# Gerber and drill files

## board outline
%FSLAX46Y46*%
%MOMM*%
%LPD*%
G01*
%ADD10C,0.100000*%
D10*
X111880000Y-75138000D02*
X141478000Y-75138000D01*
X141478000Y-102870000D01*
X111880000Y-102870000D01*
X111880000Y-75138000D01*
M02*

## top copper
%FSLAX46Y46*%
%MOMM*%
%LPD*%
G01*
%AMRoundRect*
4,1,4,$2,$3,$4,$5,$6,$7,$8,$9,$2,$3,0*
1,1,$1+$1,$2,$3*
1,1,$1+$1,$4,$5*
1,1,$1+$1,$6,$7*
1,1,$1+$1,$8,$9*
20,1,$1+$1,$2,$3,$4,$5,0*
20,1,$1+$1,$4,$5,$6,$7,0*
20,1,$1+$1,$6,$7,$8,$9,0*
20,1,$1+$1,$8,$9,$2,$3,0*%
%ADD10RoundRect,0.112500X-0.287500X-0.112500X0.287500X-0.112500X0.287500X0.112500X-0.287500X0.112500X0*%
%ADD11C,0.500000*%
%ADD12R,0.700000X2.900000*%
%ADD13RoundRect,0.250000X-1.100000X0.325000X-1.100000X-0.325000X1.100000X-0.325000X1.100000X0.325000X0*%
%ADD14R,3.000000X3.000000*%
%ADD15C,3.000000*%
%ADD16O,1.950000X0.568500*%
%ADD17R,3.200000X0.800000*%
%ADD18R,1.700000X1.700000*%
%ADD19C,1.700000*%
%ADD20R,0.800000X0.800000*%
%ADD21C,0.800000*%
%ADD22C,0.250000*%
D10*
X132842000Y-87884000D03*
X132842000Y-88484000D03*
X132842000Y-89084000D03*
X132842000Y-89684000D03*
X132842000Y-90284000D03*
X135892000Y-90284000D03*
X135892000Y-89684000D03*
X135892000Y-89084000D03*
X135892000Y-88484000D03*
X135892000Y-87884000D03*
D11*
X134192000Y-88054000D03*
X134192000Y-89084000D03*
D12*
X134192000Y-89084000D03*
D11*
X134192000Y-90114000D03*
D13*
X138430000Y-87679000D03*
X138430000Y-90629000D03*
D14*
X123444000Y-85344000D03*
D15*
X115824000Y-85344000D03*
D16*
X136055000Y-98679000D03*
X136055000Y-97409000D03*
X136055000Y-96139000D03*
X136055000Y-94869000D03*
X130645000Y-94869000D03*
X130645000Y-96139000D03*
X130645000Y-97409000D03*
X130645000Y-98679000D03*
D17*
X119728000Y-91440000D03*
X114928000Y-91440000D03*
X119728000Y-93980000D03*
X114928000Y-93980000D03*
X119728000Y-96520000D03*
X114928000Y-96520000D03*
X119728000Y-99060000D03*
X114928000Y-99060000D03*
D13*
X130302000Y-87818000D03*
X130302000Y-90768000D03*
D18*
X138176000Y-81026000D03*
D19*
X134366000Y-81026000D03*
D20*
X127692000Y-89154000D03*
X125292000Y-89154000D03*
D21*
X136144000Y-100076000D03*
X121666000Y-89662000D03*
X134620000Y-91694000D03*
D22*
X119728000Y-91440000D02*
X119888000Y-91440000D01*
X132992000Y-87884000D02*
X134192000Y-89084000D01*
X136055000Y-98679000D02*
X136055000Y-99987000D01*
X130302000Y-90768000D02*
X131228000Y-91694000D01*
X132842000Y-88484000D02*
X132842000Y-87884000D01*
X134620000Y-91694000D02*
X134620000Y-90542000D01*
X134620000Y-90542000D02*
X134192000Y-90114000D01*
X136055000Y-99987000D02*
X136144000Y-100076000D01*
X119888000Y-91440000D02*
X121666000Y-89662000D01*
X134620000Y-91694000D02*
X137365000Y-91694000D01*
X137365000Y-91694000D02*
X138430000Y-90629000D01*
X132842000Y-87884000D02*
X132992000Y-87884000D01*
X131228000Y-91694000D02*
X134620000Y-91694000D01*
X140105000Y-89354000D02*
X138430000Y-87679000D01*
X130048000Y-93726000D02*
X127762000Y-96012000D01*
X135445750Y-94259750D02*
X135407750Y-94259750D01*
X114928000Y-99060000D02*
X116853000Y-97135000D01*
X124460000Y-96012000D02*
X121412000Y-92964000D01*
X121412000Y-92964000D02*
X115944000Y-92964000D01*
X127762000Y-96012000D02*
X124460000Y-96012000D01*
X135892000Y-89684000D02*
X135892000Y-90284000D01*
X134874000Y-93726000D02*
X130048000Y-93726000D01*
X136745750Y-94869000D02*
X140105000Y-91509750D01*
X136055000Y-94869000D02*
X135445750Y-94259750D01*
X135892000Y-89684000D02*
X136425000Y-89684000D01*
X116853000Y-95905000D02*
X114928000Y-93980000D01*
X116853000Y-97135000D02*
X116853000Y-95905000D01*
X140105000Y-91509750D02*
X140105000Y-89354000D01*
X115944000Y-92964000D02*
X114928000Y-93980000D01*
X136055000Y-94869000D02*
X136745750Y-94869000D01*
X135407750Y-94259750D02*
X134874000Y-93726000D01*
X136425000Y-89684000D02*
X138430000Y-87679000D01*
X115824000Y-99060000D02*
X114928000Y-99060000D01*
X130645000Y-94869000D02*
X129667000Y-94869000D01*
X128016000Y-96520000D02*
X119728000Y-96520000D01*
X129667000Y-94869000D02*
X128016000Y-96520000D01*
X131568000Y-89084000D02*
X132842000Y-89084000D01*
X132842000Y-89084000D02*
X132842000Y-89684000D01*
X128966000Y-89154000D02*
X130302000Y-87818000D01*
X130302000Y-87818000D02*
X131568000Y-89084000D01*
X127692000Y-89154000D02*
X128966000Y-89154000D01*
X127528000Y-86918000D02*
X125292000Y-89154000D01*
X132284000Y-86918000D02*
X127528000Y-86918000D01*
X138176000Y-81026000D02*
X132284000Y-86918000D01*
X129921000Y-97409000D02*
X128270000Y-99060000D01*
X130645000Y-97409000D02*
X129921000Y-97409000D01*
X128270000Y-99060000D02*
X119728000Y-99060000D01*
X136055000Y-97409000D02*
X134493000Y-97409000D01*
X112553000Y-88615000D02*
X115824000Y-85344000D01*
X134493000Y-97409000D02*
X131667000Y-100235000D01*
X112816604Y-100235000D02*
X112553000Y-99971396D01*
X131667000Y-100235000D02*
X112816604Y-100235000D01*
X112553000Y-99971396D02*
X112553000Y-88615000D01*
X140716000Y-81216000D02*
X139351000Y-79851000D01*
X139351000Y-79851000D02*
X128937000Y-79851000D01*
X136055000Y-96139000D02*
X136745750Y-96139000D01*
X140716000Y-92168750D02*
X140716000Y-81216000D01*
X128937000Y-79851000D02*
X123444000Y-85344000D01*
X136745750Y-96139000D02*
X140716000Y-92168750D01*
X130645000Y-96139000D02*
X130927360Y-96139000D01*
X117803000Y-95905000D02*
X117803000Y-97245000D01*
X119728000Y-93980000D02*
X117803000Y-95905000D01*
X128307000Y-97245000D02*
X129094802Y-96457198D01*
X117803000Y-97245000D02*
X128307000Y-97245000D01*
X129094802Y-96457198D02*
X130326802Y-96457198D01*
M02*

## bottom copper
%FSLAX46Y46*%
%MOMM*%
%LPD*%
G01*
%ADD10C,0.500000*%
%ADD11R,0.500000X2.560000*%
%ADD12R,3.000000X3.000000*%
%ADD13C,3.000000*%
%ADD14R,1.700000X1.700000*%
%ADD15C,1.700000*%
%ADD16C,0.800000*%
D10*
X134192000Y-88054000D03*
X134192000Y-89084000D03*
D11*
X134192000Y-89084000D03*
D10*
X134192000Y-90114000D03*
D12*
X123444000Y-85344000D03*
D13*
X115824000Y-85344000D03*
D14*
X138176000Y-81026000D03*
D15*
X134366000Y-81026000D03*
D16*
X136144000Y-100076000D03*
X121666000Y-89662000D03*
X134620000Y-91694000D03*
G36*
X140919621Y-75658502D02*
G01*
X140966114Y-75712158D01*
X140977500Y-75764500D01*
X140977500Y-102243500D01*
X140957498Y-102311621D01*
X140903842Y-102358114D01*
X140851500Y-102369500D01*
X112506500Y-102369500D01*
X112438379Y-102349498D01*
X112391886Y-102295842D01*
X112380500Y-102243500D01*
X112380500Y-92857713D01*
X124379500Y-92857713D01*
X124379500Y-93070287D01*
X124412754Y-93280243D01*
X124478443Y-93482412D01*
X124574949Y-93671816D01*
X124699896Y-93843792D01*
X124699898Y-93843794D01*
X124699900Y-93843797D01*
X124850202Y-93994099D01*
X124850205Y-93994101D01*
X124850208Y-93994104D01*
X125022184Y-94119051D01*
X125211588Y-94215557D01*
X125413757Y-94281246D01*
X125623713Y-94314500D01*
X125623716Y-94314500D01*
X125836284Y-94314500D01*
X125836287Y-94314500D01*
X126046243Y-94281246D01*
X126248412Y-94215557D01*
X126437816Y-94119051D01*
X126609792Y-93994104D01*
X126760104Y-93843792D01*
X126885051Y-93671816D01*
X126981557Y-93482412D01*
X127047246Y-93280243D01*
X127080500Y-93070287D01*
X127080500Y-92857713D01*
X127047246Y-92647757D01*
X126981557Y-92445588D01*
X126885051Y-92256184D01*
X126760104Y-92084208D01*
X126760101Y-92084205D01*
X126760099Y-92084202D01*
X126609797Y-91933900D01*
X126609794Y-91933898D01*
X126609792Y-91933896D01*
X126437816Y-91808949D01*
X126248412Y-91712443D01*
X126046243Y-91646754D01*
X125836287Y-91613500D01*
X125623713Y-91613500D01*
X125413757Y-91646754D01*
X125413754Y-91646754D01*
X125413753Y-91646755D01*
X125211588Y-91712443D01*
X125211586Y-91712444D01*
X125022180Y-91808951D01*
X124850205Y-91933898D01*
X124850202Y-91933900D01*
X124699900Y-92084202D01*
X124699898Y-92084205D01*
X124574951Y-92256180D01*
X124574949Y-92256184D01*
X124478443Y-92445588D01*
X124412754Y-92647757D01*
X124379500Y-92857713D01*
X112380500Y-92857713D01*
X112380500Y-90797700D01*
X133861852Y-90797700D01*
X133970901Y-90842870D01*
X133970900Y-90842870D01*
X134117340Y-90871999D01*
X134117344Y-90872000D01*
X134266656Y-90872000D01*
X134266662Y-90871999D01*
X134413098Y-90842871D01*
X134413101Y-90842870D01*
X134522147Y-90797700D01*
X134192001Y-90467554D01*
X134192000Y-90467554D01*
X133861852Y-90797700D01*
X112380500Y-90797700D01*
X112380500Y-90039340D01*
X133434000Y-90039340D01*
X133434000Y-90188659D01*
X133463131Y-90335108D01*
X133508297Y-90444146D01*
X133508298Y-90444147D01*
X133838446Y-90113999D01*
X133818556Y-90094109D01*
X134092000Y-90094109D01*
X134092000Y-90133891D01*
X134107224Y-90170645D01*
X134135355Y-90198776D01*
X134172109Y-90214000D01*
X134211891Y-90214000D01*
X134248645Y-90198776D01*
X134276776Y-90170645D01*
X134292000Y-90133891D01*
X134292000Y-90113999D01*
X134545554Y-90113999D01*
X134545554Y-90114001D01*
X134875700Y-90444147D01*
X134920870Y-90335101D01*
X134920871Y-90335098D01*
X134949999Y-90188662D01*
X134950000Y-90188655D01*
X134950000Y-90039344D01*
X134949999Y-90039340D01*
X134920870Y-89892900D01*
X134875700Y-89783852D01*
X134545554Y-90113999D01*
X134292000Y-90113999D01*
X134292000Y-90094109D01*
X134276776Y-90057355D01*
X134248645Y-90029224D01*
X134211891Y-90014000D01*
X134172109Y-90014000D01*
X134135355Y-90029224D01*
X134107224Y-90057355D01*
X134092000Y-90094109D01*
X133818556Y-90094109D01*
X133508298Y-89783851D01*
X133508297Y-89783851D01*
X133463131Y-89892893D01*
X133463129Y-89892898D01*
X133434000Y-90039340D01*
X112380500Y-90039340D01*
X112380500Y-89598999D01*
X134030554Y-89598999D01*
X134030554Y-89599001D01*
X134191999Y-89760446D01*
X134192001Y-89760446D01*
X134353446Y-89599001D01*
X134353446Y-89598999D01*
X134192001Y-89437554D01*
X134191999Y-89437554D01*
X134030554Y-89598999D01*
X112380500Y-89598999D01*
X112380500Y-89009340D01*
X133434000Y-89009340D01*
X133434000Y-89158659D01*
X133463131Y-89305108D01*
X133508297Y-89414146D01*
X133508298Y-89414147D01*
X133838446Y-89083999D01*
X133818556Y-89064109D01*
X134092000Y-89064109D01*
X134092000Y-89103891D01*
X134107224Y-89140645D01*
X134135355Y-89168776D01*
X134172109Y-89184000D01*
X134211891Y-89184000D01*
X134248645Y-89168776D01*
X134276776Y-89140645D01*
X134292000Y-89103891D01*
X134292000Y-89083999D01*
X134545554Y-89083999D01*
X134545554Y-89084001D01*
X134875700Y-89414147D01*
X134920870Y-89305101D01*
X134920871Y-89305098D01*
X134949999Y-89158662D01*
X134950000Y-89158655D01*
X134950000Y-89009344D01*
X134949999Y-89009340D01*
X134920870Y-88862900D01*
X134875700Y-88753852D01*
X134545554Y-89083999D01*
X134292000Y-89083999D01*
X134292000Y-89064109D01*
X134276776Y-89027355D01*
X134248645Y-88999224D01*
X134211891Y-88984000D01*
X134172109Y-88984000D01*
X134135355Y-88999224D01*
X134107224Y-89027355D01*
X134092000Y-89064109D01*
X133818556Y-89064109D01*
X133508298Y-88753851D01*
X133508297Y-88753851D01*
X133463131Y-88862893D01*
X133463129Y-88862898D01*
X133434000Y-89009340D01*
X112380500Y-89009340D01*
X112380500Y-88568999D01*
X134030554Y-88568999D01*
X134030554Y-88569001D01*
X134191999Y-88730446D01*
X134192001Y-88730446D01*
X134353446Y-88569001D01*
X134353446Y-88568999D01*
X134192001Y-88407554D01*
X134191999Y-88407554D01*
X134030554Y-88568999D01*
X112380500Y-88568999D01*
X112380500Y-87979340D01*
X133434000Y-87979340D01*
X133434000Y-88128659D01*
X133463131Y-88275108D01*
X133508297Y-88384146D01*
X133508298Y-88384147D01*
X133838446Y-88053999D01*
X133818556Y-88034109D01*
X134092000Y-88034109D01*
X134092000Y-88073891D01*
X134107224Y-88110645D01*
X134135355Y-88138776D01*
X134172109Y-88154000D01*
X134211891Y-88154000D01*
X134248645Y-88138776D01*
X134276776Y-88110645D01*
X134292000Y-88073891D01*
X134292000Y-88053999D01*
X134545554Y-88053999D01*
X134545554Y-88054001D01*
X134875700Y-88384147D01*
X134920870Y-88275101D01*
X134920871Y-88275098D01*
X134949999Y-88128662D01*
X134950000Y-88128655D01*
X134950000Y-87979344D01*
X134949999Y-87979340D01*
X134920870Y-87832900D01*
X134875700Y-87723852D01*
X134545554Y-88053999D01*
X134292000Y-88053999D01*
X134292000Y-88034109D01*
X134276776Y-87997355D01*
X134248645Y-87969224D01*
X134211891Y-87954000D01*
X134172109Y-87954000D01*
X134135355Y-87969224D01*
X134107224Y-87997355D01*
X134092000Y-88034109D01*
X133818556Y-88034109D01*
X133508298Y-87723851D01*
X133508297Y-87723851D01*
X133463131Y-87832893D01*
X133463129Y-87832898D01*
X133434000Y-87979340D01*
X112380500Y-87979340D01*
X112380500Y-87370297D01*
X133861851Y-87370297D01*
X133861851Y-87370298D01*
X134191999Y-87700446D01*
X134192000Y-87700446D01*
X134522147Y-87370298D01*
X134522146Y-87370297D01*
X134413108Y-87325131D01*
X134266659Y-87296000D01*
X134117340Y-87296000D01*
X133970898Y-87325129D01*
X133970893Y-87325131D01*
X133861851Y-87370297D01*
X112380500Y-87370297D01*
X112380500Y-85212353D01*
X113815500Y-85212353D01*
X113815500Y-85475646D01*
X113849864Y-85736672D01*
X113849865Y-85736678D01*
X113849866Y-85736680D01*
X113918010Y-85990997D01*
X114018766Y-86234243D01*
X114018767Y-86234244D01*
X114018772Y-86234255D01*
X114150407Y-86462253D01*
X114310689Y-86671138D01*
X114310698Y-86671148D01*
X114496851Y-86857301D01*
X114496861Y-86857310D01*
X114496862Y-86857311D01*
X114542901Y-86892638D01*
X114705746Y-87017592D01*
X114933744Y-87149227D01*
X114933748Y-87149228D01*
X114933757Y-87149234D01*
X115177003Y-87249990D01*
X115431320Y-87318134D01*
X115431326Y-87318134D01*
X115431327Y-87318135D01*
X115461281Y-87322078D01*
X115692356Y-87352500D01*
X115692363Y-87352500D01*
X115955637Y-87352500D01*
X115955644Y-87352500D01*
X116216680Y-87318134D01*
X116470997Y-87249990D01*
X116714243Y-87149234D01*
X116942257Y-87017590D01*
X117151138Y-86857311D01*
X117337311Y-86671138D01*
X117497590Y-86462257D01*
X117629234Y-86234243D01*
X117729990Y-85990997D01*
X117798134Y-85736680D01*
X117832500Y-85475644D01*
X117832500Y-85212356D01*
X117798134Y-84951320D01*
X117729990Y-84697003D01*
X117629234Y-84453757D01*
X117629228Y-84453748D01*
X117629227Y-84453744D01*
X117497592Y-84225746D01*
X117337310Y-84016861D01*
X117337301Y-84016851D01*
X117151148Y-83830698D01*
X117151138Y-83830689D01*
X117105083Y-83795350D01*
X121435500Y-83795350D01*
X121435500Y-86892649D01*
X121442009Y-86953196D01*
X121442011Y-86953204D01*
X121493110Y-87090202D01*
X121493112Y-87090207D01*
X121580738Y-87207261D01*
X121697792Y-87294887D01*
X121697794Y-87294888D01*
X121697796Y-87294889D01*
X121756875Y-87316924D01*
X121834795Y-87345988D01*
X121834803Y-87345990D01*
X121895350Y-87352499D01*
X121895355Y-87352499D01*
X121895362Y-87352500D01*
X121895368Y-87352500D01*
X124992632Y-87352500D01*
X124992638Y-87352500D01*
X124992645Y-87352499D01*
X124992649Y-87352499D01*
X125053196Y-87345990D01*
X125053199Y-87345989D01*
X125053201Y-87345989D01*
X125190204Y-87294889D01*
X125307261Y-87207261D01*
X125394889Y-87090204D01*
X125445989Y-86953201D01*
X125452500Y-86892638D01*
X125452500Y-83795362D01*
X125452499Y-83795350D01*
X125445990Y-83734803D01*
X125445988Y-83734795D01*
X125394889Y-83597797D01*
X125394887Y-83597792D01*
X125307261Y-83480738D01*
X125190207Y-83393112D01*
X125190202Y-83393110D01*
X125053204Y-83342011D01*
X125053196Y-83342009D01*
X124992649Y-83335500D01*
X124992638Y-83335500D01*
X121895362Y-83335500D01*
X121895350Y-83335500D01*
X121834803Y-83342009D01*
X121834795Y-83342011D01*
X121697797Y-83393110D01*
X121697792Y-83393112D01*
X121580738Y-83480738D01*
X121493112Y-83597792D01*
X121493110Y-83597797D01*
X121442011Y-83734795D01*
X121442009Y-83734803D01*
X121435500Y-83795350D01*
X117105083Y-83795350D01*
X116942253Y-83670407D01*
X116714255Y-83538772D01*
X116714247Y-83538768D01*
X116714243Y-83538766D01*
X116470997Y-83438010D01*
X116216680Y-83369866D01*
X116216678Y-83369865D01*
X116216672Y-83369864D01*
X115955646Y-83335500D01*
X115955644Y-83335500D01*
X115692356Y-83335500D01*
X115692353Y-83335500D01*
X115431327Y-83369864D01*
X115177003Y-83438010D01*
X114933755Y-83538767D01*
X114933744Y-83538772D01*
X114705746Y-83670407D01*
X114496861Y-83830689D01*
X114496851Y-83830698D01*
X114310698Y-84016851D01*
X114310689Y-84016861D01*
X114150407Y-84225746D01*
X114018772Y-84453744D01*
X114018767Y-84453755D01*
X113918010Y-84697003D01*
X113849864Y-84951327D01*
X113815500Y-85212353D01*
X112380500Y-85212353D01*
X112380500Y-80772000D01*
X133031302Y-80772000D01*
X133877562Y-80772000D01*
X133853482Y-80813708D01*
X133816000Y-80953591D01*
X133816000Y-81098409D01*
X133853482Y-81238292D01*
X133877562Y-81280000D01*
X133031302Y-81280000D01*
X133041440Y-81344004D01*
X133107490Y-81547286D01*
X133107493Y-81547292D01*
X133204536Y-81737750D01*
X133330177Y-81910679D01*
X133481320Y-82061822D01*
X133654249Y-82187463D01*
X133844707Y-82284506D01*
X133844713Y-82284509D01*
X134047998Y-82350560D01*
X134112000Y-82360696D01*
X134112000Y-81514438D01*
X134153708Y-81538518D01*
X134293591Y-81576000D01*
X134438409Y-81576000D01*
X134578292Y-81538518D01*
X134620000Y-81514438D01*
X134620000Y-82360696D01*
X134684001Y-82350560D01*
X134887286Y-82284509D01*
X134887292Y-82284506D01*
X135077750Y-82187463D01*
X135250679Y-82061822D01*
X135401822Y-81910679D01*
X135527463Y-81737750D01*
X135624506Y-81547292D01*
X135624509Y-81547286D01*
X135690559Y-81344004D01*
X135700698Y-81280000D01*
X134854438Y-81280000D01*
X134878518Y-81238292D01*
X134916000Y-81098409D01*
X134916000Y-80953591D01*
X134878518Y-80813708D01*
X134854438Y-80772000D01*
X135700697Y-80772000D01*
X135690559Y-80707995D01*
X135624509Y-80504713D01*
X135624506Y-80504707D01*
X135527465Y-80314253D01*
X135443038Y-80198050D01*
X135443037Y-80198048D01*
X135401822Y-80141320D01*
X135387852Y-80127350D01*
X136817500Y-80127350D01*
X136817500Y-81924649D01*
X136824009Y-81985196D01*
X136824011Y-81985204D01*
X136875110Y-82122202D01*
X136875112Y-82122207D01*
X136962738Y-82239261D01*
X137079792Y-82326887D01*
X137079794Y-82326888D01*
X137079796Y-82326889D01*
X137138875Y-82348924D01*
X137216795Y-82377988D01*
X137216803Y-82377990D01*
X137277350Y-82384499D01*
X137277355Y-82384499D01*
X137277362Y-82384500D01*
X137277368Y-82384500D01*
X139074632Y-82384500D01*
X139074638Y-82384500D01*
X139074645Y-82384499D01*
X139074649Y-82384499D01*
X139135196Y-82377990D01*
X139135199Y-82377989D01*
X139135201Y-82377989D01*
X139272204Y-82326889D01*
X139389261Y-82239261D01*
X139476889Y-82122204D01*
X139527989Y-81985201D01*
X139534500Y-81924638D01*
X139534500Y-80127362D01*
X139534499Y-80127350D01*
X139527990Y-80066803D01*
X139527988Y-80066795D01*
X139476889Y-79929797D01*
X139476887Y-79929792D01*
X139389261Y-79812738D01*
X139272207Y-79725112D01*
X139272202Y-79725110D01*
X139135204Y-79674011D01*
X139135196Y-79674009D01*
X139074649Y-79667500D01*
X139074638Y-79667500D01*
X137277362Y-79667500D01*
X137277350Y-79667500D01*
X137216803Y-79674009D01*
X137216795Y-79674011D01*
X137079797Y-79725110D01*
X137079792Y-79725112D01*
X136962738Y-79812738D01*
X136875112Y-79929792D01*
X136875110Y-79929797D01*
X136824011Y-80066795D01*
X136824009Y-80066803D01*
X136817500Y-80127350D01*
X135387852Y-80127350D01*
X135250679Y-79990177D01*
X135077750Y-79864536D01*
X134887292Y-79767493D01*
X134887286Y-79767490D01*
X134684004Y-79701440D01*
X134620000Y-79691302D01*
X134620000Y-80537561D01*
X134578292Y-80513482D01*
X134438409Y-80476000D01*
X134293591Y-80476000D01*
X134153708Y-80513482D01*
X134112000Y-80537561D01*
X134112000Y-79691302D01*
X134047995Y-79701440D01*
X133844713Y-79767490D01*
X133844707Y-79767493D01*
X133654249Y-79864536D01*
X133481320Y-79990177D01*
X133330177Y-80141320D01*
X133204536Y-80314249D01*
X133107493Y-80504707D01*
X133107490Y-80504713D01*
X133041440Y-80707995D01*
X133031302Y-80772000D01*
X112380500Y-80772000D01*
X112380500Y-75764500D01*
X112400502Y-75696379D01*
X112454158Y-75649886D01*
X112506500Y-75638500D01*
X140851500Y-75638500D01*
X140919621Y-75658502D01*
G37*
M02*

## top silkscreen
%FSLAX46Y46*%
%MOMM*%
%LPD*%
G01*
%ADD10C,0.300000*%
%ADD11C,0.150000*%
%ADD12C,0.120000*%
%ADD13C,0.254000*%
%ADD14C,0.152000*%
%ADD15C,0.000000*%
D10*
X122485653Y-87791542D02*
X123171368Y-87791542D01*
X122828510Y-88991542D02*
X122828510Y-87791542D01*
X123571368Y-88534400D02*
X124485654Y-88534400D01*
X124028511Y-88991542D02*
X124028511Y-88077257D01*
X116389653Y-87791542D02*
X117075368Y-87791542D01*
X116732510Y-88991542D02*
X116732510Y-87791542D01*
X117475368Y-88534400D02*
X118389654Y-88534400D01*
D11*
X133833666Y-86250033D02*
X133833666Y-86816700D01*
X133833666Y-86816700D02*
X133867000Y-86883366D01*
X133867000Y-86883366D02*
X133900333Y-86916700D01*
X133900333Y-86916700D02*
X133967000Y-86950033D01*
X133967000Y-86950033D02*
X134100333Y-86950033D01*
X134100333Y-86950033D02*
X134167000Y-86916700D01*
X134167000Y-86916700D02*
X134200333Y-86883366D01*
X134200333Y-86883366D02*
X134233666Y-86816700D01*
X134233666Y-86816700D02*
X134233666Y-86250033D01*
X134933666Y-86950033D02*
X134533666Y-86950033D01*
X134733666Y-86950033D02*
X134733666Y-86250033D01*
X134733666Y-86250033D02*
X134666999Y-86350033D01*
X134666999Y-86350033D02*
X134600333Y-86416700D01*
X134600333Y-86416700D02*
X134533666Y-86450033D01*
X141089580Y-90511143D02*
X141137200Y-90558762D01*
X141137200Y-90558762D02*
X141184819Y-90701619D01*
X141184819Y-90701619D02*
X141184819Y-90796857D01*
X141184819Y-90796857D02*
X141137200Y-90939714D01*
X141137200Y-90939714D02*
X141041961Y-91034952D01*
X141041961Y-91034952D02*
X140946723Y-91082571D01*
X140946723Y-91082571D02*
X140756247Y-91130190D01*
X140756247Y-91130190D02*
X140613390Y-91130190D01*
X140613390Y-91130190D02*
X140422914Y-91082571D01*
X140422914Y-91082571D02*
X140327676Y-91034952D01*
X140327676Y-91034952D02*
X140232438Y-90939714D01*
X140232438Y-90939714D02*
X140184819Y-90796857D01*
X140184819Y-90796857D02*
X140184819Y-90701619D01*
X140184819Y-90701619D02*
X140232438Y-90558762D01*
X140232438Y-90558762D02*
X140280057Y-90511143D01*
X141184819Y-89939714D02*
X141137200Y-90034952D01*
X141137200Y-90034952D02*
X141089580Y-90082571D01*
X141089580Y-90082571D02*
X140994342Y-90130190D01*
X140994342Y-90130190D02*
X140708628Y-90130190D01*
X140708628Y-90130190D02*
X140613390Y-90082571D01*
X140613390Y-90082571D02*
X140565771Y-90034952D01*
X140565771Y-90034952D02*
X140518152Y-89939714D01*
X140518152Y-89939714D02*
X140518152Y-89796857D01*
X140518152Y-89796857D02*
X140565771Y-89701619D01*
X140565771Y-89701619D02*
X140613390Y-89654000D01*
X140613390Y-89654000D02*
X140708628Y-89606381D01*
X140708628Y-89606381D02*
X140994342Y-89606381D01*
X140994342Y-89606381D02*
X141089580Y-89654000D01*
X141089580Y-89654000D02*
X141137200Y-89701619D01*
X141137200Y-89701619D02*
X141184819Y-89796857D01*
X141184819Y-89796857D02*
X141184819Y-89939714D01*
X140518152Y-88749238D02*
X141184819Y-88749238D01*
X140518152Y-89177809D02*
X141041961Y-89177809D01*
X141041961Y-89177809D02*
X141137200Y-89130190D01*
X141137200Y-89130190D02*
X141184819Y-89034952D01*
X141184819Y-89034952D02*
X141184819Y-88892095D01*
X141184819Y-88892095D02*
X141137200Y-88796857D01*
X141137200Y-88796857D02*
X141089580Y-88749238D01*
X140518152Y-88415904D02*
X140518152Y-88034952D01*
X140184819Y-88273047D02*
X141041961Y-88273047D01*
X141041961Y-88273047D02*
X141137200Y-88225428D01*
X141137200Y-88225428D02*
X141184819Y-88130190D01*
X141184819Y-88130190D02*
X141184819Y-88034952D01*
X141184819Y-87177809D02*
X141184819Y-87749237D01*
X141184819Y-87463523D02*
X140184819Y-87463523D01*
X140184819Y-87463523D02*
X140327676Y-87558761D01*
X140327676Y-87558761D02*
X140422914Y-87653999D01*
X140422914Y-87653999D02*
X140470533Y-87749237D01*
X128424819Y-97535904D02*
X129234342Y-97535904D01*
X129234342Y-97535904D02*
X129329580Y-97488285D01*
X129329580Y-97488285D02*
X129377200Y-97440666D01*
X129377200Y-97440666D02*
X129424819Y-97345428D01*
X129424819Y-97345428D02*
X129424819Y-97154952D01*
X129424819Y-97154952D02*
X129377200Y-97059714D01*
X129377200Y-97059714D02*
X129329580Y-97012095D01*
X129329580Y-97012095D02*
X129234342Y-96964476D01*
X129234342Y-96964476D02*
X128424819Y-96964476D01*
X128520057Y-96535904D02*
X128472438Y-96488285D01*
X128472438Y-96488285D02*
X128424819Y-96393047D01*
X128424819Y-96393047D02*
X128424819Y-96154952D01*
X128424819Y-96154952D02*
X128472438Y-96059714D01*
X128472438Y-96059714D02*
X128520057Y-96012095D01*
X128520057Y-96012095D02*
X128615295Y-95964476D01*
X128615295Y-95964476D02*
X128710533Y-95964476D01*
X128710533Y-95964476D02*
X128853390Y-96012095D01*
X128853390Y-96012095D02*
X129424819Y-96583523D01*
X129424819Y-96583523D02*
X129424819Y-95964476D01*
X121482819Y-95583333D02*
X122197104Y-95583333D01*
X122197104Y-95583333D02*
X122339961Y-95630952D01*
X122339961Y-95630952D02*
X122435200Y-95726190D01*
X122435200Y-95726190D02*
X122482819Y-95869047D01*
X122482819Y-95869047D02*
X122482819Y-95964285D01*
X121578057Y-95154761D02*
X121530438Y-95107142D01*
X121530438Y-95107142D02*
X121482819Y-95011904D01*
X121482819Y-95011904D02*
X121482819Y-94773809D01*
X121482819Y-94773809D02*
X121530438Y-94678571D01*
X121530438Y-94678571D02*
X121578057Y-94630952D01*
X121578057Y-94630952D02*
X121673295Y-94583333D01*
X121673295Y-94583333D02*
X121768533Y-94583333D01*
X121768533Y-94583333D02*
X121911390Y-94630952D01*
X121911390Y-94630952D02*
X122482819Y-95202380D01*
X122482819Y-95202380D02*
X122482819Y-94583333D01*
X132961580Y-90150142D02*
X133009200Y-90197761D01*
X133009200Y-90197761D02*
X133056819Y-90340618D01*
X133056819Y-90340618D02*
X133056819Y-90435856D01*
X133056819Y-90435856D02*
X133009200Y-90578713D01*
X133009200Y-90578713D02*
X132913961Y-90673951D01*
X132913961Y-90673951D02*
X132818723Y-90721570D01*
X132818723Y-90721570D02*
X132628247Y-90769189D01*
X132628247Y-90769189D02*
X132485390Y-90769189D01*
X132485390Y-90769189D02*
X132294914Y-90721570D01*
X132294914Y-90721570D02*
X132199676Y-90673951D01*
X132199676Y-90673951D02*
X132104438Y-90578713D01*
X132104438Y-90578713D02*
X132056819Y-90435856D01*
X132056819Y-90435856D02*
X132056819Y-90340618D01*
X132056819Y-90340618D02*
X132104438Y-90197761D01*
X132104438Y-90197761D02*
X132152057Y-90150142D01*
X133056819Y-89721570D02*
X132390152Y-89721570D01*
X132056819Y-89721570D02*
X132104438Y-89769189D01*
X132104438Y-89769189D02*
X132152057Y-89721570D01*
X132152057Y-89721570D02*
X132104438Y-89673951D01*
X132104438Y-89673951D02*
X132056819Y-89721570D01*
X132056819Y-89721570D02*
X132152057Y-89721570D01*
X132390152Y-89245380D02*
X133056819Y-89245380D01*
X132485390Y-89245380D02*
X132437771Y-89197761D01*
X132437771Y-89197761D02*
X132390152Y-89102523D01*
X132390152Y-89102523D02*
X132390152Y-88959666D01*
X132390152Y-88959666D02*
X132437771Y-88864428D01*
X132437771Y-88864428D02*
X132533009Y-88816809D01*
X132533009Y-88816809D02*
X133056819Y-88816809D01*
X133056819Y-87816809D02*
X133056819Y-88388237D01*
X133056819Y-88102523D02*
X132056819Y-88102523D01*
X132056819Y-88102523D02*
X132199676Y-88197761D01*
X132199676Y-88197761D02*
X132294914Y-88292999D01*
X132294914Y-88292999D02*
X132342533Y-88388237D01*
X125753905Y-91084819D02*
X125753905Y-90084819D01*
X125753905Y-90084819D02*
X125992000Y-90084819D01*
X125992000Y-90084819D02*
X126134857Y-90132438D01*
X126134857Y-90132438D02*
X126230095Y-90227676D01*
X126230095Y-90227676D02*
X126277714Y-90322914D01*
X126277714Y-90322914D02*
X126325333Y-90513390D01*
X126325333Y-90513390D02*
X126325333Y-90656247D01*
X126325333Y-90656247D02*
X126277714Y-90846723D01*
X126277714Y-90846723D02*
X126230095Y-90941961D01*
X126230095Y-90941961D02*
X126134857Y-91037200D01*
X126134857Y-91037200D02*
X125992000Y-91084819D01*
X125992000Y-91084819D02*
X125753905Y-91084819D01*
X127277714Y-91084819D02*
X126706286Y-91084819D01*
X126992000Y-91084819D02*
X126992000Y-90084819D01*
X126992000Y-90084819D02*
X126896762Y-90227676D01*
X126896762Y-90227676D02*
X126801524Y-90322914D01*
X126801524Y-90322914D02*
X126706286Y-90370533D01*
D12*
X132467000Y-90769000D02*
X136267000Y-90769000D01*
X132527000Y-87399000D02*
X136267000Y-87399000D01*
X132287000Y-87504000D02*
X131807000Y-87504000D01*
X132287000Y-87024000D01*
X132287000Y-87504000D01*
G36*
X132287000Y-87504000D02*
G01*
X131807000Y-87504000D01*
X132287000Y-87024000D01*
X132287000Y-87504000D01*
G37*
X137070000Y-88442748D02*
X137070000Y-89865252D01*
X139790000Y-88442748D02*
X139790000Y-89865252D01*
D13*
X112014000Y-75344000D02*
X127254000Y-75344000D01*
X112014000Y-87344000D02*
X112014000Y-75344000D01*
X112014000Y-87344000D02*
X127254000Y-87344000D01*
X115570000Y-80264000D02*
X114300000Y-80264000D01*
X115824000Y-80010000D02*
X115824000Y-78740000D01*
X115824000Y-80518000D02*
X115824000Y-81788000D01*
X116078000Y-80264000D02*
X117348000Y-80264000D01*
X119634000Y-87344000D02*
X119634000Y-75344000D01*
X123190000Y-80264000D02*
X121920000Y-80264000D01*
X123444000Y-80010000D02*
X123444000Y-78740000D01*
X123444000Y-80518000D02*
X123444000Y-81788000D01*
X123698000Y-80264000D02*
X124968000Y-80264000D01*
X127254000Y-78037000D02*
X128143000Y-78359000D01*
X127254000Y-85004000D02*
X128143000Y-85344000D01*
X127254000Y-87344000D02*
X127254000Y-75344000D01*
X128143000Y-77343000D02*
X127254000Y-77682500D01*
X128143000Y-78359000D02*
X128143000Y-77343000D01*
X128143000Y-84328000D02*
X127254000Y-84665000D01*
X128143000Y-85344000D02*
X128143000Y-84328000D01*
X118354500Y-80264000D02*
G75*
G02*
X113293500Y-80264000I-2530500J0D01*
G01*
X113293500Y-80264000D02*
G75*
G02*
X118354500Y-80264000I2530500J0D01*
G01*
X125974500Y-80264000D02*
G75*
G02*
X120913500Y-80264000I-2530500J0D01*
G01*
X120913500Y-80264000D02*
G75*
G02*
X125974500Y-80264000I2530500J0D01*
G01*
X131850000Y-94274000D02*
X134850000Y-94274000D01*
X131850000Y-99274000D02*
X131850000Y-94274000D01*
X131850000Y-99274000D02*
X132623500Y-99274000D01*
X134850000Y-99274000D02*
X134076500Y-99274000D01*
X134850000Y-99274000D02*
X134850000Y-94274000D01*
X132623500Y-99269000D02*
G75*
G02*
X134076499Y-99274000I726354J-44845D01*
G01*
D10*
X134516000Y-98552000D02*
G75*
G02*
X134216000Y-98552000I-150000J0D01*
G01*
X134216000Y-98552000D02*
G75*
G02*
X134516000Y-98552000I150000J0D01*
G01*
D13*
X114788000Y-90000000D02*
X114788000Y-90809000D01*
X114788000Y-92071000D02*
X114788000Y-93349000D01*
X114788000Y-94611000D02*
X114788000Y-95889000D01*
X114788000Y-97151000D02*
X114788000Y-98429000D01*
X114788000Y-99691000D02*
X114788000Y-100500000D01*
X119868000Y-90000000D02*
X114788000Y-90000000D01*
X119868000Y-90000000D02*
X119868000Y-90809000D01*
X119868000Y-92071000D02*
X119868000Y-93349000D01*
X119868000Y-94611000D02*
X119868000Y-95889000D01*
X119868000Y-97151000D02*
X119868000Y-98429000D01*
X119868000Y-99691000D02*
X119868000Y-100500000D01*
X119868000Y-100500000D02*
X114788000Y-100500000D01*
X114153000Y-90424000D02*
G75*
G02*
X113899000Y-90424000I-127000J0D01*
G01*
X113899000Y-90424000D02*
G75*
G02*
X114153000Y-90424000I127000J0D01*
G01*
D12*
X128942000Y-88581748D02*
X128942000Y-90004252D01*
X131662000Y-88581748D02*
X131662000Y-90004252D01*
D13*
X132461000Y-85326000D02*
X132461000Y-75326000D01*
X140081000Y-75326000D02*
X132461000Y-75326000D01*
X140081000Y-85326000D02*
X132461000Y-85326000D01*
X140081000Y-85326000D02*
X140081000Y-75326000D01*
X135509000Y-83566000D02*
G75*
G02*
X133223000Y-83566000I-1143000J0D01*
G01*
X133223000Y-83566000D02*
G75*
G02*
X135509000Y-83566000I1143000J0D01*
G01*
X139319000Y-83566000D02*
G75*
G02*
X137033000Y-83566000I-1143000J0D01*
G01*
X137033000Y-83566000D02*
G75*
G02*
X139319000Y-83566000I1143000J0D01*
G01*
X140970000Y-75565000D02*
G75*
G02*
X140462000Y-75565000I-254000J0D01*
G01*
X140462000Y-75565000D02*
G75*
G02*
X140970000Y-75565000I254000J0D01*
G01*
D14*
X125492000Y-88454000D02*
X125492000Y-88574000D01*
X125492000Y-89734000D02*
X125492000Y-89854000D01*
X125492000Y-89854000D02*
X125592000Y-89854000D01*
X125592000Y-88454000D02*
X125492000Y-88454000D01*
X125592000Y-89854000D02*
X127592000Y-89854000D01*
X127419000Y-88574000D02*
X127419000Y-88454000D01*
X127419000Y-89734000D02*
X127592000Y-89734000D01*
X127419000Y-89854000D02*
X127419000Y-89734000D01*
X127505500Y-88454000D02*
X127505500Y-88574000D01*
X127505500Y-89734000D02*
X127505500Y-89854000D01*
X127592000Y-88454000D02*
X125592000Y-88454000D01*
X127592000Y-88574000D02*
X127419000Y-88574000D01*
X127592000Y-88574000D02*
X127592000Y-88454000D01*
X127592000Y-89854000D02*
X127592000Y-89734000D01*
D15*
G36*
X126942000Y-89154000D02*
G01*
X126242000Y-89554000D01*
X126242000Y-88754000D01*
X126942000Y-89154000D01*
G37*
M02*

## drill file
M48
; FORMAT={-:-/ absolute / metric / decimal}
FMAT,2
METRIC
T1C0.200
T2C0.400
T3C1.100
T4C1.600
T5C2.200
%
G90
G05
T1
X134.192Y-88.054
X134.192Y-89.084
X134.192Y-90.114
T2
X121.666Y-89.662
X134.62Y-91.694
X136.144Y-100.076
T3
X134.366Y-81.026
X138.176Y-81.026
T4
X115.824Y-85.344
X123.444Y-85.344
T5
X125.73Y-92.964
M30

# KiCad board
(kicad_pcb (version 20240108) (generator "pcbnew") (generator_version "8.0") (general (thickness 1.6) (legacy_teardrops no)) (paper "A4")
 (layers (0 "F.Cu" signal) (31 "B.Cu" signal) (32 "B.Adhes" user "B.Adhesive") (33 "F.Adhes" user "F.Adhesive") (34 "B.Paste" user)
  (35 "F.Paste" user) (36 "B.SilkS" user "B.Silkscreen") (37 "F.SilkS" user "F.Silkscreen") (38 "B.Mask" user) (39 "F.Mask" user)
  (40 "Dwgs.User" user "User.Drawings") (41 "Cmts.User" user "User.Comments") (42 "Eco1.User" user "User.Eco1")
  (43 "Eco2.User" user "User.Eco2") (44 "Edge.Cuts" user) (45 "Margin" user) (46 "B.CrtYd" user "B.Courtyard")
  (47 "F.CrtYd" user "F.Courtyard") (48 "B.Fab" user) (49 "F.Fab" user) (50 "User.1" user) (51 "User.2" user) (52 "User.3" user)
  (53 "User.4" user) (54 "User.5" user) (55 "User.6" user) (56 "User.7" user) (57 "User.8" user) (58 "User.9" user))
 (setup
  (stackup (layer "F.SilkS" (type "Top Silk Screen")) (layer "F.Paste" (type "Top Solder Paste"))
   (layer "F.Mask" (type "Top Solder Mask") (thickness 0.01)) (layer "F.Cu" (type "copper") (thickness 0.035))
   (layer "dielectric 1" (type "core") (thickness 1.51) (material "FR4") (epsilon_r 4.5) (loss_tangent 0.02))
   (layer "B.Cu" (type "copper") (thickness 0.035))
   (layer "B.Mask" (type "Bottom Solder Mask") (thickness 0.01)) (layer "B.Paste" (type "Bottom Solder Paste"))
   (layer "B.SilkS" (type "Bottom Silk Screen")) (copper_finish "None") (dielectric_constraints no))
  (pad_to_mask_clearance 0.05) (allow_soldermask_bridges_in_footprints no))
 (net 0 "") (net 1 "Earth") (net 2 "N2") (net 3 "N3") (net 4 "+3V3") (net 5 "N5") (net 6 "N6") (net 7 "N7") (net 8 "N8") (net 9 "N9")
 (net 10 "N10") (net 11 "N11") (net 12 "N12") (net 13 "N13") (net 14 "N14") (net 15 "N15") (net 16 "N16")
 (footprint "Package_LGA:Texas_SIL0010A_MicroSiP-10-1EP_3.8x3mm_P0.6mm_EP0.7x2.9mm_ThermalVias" (layer "F.Cu") (at 134.367 89.084)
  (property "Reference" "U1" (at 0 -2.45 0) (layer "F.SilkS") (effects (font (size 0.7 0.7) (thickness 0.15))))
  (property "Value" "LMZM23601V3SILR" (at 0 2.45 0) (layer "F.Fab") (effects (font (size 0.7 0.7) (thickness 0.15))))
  (fp_line (start -1.9 1.685) (end 1.9 1.685) (stroke (width 0.12) (type solid)) (layer "F.SilkS"))
  (fp_line (start -1.84 -1.685) (end 1.9 -1.685) (stroke (width 0.12) (type solid)) (layer "F.SilkS"))
  (fp_poly
   (pts (xy -2.08 -1.58) (xy -2.56 -1.58) (xy -2.08 -2.06) (xy -2.08 -1.58)) (stroke (width 0.12) (type solid)) (fill solid)
   (layer "F.SilkS"))
  (pad "" smd roundrect (at -0.175 -0.97) (size 0.65 0.9) (layers "F.Paste") (roundrect_rratio 0.25))
  (pad "" smd roundrect (at -0.175 0) (size 0.65 0.9) (layers "F.Paste") (roundrect_rratio 0.25))
  (pad "" smd roundrect (at -0.175 0.97) (size 0.65 0.9) (layers "F.Paste") (roundrect_rratio 0.25))
  (pad "1" smd roundrect (at -1.525 -1.2) (size 0.8 0.45) (layers "F.Cu" "F.Paste" "F.Mask") (roundrect_rratio 0.25) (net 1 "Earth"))
  (pad "2" smd roundrect (at -1.525 -0.6) (size 0.8 0.45) (layers "F.Cu" "F.Paste" "F.Mask") (roundrect_rratio 0.25) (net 1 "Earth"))
  (pad "3" smd roundrect (at -1.525 0) (size 0.8 0.45) (layers "F.Cu" "F.Paste" "F.Mask") (roundrect_rratio 0.25) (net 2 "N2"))
  (pad "4" smd roundrect (at -1.525 0.6) (size 0.8 0.45) (layers "F.Cu" "F.Paste" "F.Mask") (roundrect_rratio 0.25) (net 2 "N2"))
  (pad "5" smd roundrect (at -1.525 1.2) (size 0.8 0.45) (layers "F.Cu" "F.Paste" "F.Mask") (roundrect_rratio 0.25) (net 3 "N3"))
  (pad "6" smd roundrect (at 1.525 1.2) (size 0.8 0.45) (layers "F.Cu" "F.Paste" "F.Mask") (roundrect_rratio 0.25) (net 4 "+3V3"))
  (pad "7" smd roundrect (at 1.525 0.6) (size 0.8 0.45) (layers "F.Cu" "F.Paste" "F.Mask") (roundrect_rratio 0.25) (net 4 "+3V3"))
  (pad "8" smd roundrect (at 1.525 0) (size 0.8 0.45) (layers "F.Cu" "F.Paste" "F.Mask") (roundrect_rratio 0.25) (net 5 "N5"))
  (pad "9" smd roundrect (at 1.525 -0.6) (size 0.8 0.45) (layers "F.Cu" "F.Paste" "F.Mask") (roundrect_rratio 0.25) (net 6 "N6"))
  (pad "10" smd roundrect (at 1.525 -1.2) (size 0.8 0.45) (layers "F.Cu" "F.Paste" "F.Mask") (roundrect_rratio 0.25) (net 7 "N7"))
  (pad "11" thru_hole circle (at -0.175 -1.03) (size 0.5 0.5) (drill 0.2) (layers "*.Cu") (remove_unused_layers no) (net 1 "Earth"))
  (pad "11" thru_hole circle (at -0.175 0) (size 0.5 0.5) (drill 0.2) (layers "*.Cu") (remove_unused_layers no) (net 1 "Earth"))
  (pad "11" smd rect (at -0.175 0) (size 0.5 2.56) (layers "B.Cu") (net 1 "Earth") (zone_connect 2))
  (pad "11" smd rect (at -0.175 0) (size 0.7 2.9) (layers "F.Cu" "F.Mask") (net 1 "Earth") (zone_connect 2))
  (pad "11" thru_hole circle (at -0.175 1.03) (size 0.5 0.5) (drill 0.2) (layers "*.Cu") (remove_unused_layers no) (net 1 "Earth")))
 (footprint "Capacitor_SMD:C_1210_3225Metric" (layer "F.Cu") (at 138.43 89.154 -90)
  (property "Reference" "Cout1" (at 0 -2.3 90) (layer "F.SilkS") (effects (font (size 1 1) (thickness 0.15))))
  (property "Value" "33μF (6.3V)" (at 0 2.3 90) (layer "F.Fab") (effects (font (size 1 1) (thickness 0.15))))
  (fp_line (start -0.711252 1.36) (end 0.711252 1.36) (stroke (width 0.12) (type solid)) (layer "F.SilkS"))
  (fp_line (start -0.711252 -1.36) (end 0.711252 -1.36) (stroke (width 0.12) (type solid)) (layer "F.SilkS"))
  (pad "1" smd roundrect (at -1.475 0 270) (size 1.15 2.7) (layers "F.Cu" "F.Paste" "F.Mask") (roundrect_rratio 0.217391) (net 4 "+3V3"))
  (pad "2" smd roundrect (at 1.475 0 270) (size 1.15 2.7) (layers "F.Cu" "F.Paste" "F.Mask") (roundrect_rratio 0.217391) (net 1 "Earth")))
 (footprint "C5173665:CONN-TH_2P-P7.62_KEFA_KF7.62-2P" (layer "F.Cu") (at 119.634 85.344 180)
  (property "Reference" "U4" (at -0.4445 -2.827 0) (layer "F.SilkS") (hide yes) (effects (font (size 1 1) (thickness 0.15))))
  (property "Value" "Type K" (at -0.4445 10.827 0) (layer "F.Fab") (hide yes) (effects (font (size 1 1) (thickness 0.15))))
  (fp_line (start 7.62 10) (end -7.62 10) (stroke (width 0.254) (type default)) (layer "F.SilkS"))
  (fp_line (start 7.62 -2) (end 7.62 10) (stroke (width 0.254) (type default)) (layer "F.SilkS"))
  (fp_line (start 7.62 -2) (end -7.62 -2) (stroke (width 0.254) (type default)) (layer "F.SilkS"))
  (fp_line (start 4.064 5.08) (end 5.334 5.08) (stroke (width 0.254) (type default)) (layer "F.SilkS"))
  (fp_line (start 3.81 5.334) (end 3.81 6.604) (stroke (width 0.254) (type default)) (layer "F.SilkS"))
  (fp_line (start 3.81 4.826) (end 3.81 3.556) (stroke (width 0.254) (type default)) (layer "F.SilkS"))
  (fp_line (start 3.556 5.08) (end 2.286 5.08) (stroke (width 0.254) (type default)) (layer "F.SilkS"))
  (fp_line (start 0 -2) (end 0 10) (stroke (width 0.254) (type default)) (layer "F.SilkS"))
  (fp_line (start -3.556 5.08) (end -2.286 5.08) (stroke (width 0.254) (type default)) (layer "F.SilkS"))
  (fp_line (start -3.81 5.334) (end -3.81 6.604) (stroke (width 0.254) (type default)) (layer "F.SilkS"))
  (fp_line (start -3.81 4.826) (end -3.81 3.556) (stroke (width 0.254) (type default)) (layer "F.SilkS"))
  (fp_line (start -4.064 5.08) (end -5.334 5.08) (stroke (width 0.254) (type default)) (layer "F.SilkS"))
  (fp_line (start -7.62 7.307) (end -8.509 6.985) (stroke (width 0.254) (type default)) (layer "F.SilkS"))
  (fp_line (start -7.62 0.34) (end -8.509 0) (stroke (width 0.254) (type default)) (layer "F.SilkS"))
  (fp_line (start -7.62 -2) (end -7.62 10) (stroke (width 0.254) (type default)) (layer "F.SilkS"))
  (fp_line (start -8.509 8.001) (end -7.62 7.6615) (stroke (width 0.254) (type default)) (layer "F.SilkS"))
  (fp_line (start -8.509 6.985) (end -8.509 8.001) (stroke (width 0.254) (type default)) (layer "F.SilkS"))
  (fp_line (start -8.509 1.016) (end -7.62 0.679) (stroke (width 0.254) (type default)) (layer "F.SilkS"))
  (fp_line (start -8.509 0) (end -8.509 1.016) (stroke (width 0.254) (type default)) (layer "F.SilkS"))
  (fp_circle (center 3.81 5.08) (end 6.3405 5.08) (stroke (width 0.254) (type default)) (fill none) (layer "F.SilkS"))
  (fp_circle (center -3.81 5.08) (end -1.2795 5.08) (stroke (width 0.254) (type default)) (fill none) (layer "F.SilkS"))
  (pad "1" thru_hole rect (at -3.81 0 180) (size 3 3) (drill 1.6) (layers "*.Cu" "*.Mask") (remove_unused_layers no) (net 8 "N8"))
  (pad "2" thru_hole circle (at 3.81 0 180) (size 3 3) (drill 1.6) (layers "*.Cu" "*.Mask") (remove_unused_layers no) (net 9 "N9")
   (thermal_bridge_angle 90)))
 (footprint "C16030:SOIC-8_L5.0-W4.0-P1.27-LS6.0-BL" (layer "F.Cu") (at 133.35 96.774 90)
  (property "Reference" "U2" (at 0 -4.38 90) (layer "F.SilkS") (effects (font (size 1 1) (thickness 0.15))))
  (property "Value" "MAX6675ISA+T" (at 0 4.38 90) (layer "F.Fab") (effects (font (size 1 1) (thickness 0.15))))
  (fp_line (start 2.5 -1.5) (end 2.5 1.5) (stroke (width 0.254) (type default)) (layer "F.SilkS"))
  (fp_line (start -2.5 -1.5) (end 2.5 -1.5) (stroke (width 0.254) (type default)) (layer "F.SilkS"))
  (fp_line (start -2.5 -1.5) (end -2.5 -0.7265) (stroke (width 0.254) (type default)) (layer "F.SilkS"))
  (fp_line (start -2.5 1.5) (end -2.5 0.7265) (stroke (width 0.254) (type default)) (layer "F.SilkS"))
  (fp_line (start -2.5 1.5) (end 2.5 1.5) (stroke (width 0.254) (type default)) (layer "F.SilkS"))
  (fp_arc (start -2.495 -0.7265) (mid -1.812112 0.002358) (end -2.5 0.7265) (stroke (width 0.254) (type default)) (layer "F.SilkS"))
  (fp_circle (center -1.778 1.016) (end -1.628 1.016) (stroke (width 0.3) (type default)) (fill none) (layer "F.SilkS"))
  (pad "1" smd oval (at -1.905 2.705 90) (size 0.5685 1.95) (layers "F.Cu" "F.Paste" "F.Mask") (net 1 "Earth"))
  (pad "2" smd oval (at -0.635 2.705 90) (size 0.5685 1.95) (layers "F.Cu" "F.Paste" "F.Mask") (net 9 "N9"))
  (pad "3" smd oval (at 0.635 2.705 90) (size 0.5685 1.95) (layers "F.Cu" "F.Paste" "F.Mask") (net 8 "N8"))
  (pad "4" smd oval (at 1.905 2.705 90) (size 0.5685 1.95) (layers "F.Cu" "F.Paste" "F.Mask") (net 4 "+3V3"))
  (pad "5" smd oval (at 1.905 -2.705 90) (size 0.5685 1.95) (layers "F.Cu" "F.Paste" "F.Mask") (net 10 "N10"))
  (pad "6" smd oval (at 0.635 -2.705 90) (size 0.5685 1.95) (layers "F.Cu" "F.Paste" "F.Mask") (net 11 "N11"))
  (pad "7" smd oval (at -0.635 -2.705 90) (size 0.5685 1.95) (layers "F.Cu" "F.Paste" "F.Mask") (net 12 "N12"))
  (pad "8" smd oval (at -1.905 -2.705 90) (size 0.5685 1.95) (layers "F.Cu" "F.Paste" "F.Mask") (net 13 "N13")))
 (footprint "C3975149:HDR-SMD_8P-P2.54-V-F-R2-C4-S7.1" (layer "F.Cu") (at 117.328 95.25 -90)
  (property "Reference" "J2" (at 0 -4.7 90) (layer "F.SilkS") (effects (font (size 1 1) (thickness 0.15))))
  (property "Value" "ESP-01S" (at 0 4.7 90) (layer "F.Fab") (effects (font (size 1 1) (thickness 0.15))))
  (fp_line (start -5.25 2.54) (end -4.441 2.54) (stroke (width 0.254) (type default)) (layer "F.SilkS"))
  (fp_line (start -3.179 2.54) (end -1.901 2.54) (stroke (width 0.254) (type default)) (layer "F.SilkS"))
  (fp_line (start -0.639 2.54) (end 0.639 2.54) (stroke (width 0.254) (type default)) (layer "F.SilkS"))
  (fp_line (start 1.901 2.54) (end 3.179 2.54) (stroke (width 0.254) (type default)) (layer "F.SilkS"))
  (fp_line (start 4.441 2.54) (end 5.25 2.54) (stroke (width 0.254) (type default)) (layer "F.SilkS"))
  (fp_line (start -5.25 -2.54) (end -5.25 2.54) (stroke (width 0.254) (type default)) (layer "F.SilkS"))
  (fp_line (start -5.25 -2.54) (end -4.441 -2.54) (stroke (width 0.254) (type default)) (layer "F.SilkS"))
  (fp_line (start -3.179 -2.54) (end -1.901 -2.54) (stroke (width 0.254) (type default)) (layer "F.SilkS"))
  (fp_line (start -0.639 -2.54) (end 0.639 -2.54) (stroke (width 0.254) (type default)) (layer "F.SilkS"))
  (fp_line (start 1.901 -2.54) (end 3.179 -2.54) (stroke (width 0.254) (type default)) (layer "F.SilkS"))
  (fp_line (start 4.441 -2.54) (end 5.25 -2.54) (stroke (width 0.254) (type default)) (layer "F.SilkS"))
  (fp_line (start 5.25 -2.54) (end 5.25 2.54) (stroke (width 0.254) (type default)) (layer "F.SilkS"))
  (fp_circle (center -4.826 3.302) (end -4.699 3.302) (stroke (width 0.254) (type default)) (fill none) (layer "F.SilkS"))
  (pad "1" smd rect (at -3.81 -2.4 270) (size 0.8 3.2) (layers "F.Cu" "F.Paste" "F.Mask") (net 1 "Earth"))
  (pad "2" smd rect (at -3.81 2.4 270) (size 0.8 3.2) (layers "F.Cu" "F.Paste" "F.Mask") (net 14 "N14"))
  (pad "3" smd rect (at -1.27 -2.4 270) (size 0.8 3.2) (layers "F.Cu" "F.Paste" "F.Mask") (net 11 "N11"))
  (pad "4" smd rect (at -1.27 2.4 270) (size 0.8 3.2) (layers "F.Cu" "F.Paste" "F.Mask") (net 4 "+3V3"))
  (pad "5" smd rect (at 1.27 -2.4 270) (size 0.8 3.2) (layers "F.Cu" "F.Paste" "F.Mask") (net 10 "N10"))
  (pad "6" smd rect (at 1.27 2.4 270) (size 0.8 3.2) (layers "F.Cu" "F.Paste" "F.Mask") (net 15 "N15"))
  (pad "7" smd rect (at 3.81 -2.4 270) (size 0.8 3.2) (layers "F.Cu" "F.Paste" "F.Mask") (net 12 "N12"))
  (pad "8" smd rect (at 3.81 2.4 270) (size 0.8 3.2) (layers "F.Cu" "F.Paste" "F.Mask") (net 4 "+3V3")))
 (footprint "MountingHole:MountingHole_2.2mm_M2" (layer "F.Cu") (at 125.73 92.964)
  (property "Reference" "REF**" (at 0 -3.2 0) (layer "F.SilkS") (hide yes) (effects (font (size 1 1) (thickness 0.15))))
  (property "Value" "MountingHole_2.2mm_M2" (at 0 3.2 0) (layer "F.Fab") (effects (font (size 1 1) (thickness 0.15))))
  (pad "" np_thru_hole circle (at 0 0) (size 2.2 2.2) (drill 2.2) (layers "*.Cu" "*.Mask")))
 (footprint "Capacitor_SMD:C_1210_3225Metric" (layer "F.Cu") (at 130.302 89.293 -90)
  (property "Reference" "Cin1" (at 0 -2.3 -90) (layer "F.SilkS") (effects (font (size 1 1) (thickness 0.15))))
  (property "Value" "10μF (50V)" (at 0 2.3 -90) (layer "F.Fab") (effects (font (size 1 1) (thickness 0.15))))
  (fp_line (start -0.711252 1.36) (end 0.711252 1.36) (stroke (width 0.12) (type solid)) (layer "F.SilkS"))
  (fp_line (start -0.711252 -1.36) (end 0.711252 -1.36) (stroke (width 0.12) (type solid)) (layer "F.SilkS"))
  (pad "1" smd roundrect (at -1.475 0 270) (size 1.15 2.7) (layers "F.Cu" "F.Paste" "F.Mask") (roundrect_rratio 0.217391) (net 2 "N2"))
  (pad "2" smd roundrect (at 1.475 0 270) (size 1.15 2.7) (layers "F.Cu" "F.Paste" "F.Mask") (roundrect_rratio 0.217391) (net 1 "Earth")))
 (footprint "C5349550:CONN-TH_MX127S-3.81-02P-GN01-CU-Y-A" (layer "F.Cu") (at 136.271 81.026 180)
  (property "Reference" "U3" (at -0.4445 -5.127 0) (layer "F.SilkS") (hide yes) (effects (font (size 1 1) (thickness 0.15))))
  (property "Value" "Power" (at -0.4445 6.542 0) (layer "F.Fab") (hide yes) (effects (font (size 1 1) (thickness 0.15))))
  (fp_line (start 3.81 -4.3) (end 3.81 5.7) (stroke (width 0.254) (type default)) (layer "F.SilkS"))
  (fp_line (start -3.81 5.7) (end 3.81 5.7) (stroke (width 0.254) (type default)) (layer "F.SilkS"))
  (fp_line (start -3.81 -4.3) (end 3.81 -4.3) (stroke (width 0.254) (type default)) (layer "F.SilkS"))
  (fp_line (start -3.81 -4.3) (end -3.81 5.7) (stroke (width 0.254) (type default)) (layer "F.SilkS"))
  (fp_circle (center 1.905 -2.54) (end 3.048 -2.54) (stroke (width 0.254) (type default)) (fill none) (layer "F.SilkS"))
  (fp_circle (center -1.905 -2.54) (end -0.762 -2.54) (stroke (width 0.254) (type default)) (fill none) (layer "F.SilkS"))
  (fp_circle (center -4.445 5.461) (end -4.191 5.461) (stroke (width 0.254) (type default)) (fill none) (layer "F.SilkS"))
  (pad "1" thru_hole rect (at -1.905 0 180) (size 1.7 1.7) (drill 1.1) (layers "*.Cu" "*.Mask") (remove_unused_layers no) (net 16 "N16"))
  (pad "2" thru_hole circle (at 1.905 0 180) (size 1.7 1.7) (drill 1.1) (layers "*.Cu" "*.Mask") (remove_unused_layers no) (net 1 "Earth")
   (thermal_bridge_angle 90)))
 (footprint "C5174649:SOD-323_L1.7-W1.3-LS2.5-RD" (layer "F.Cu") (at 126.492 89.154 180)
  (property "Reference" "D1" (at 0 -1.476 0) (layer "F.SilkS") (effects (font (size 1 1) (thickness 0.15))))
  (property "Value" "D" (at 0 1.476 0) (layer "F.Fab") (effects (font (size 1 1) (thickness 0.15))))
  (fp_line (start 1 0.7) (end 1 0.58) (stroke (width 0.152) (type default)) (layer "F.SilkS"))
  (fp_line (start 1 -0.58) (end 1 -0.7) (stroke (width 0.152) (type default)) (layer "F.SilkS"))
  (fp_line (start 1 -0.7) (end 0.9 -0.7) (stroke (width 0.152) (type default)) (layer "F.SilkS"))
  (fp_line (start 0.9 0.7) (end 1 0.7) (stroke (width 0.152) (type default)) (layer "F.SilkS"))
  (fp_line (start 0.9 -0.7) (end -1.1 -0.7) (stroke (width 0.152) (type default)) (layer "F.SilkS"))
  (fp_line (start -0.927 0.58) (end -0.927 0.7) (stroke (width 0.152) (type default)) (layer "F.SilkS"))
  (fp_line (start -0.927 -0.58) (end -1.1 -0.58) (stroke (width 0.152) (type default)) (layer "F.SilkS"))
  (fp_line (start -0.927 -0.7) (end -0.927 -0.58) (stroke (width 0.152) (type default)) (layer "F.SilkS"))
  (fp_line (start -1.0135 0.7) (end -1.0135 0.58) (stroke (width 0.152) (type default)) (layer "F.SilkS"))
  (fp_line (start -1.0135 -0.58) (end -1.0135 -0.7) (stroke (width 0.152) (type default)) (layer "F.SilkS"))
  (fp_line (start -1.1 0.7) (end 0.9 0.7) (stroke (width 0.152) (type default)) (layer "F.SilkS"))
  (fp_line (start -1.1 0.58) (end -0.927 0.58) (stroke (width 0.152) (type default)) (layer "F.SilkS"))
  (fp_line (start -1.1 0.58) (end -1.1 0.7) (stroke (width 0.152) (type default)) (layer "F.SilkS"))
  (fp_line (start -1.1 -0.7) (end -1.1 -0.58) (stroke (width 0.152) (type default)) (layer "F.SilkS"))
  (fp_poly (pts (xy -0.45 0) (xy 0.25 -0.4) (xy 0.25 0.4)) (stroke (width 0) (type default)) (fill solid) (layer "F.SilkS"))
  (pad "1" smd rect (at -1.2 0 180) (size 0.8 0.8) (layers "F.Cu" "F.Paste" "F.Mask") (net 2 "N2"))
  (pad "2" smd rect (at 1.2 0 180) (size 0.8 0.8) (layers "F.Cu" "F.Paste" "F.Mask") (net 16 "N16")))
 (gr_rect (start 111.88 75.138) (end 141.478 102.87) (stroke (width 0.1) (type solid)) (fill none) (layer "Edge.Cuts"))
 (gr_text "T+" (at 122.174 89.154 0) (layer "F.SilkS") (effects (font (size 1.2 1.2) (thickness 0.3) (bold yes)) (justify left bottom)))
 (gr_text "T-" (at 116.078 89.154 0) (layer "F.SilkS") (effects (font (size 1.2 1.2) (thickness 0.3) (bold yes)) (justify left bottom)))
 (segment (start 119.728 91.44) (end 119.888 91.44) (width 0.25) (layer "F.Cu") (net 1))
 (segment (start 132.992 87.884) (end 134.192 89.084) (width 0.25) (layer "F.Cu") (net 1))
 (segment (start 136.055 98.679) (end 136.055 99.987) (width 0.25) (layer "F.Cu") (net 1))
 (segment (start 130.302 90.768) (end 131.228 91.694) (width 0.25) (layer "F.Cu") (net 1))
 (segment (start 132.842 88.484) (end 132.842 87.884) (width 0.25) (layer "F.Cu") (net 1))
 (segment (start 134.62 91.694) (end 134.62 90.542) (width 0.25) (layer "F.Cu") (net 1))
 (segment (start 134.62 90.542) (end 134.192 90.114) (width 0.25) (layer "F.Cu") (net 1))
 (segment (start 136.055 99.987) (end 136.144 100.076) (width 0.25) (layer "F.Cu") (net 1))
 (segment (start 119.888 91.44) (end 121.666 89.662) (width 0.25) (layer "F.Cu") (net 1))
 (segment (start 134.62 91.694) (end 137.365 91.694) (width 0.25) (layer "F.Cu") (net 1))
 (segment (start 137.365 91.694) (end 138.43 90.629) (width 0.25) (layer "F.Cu") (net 1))
 (segment (start 132.842 87.884) (end 132.992 87.884) (width 0.25) (layer "F.Cu") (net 1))
 (segment (start 131.228 91.694) (end 134.62 91.694) (width 0.25) (layer "F.Cu") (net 1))
 (via (at 136.144 100.076) (size 0.8) (drill 0.4) (layers "F.Cu" "B.Cu") (free yes) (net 1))
 (via (at 121.666 89.662) (size 0.8) (drill 0.4) (layers "F.Cu" "B.Cu") (free yes) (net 1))
 (via (at 134.62 91.694) (size 0.8) (drill 0.4) (layers "F.Cu" "B.Cu") (free yes) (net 1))
 (segment (start 140.105 89.354) (end 138.43 87.679) (width 0.25) (layer "F.Cu") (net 4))
 (segment (start 130.048 93.726) (end 127.762 96.012) (width 0.25) (layer "F.Cu") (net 4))
 (segment (start 135.44575 94.25975) (end 135.40775 94.25975) (width 0.25) (layer "F.Cu") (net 4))
 (segment (start 114.928 99.06) (end 116.853 97.135) (width 0.25) (layer "F.Cu") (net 4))
 (segment (start 124.46 96.012) (end 121.412 92.964) (width 0.25) (layer "F.Cu") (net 4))
 (segment (start 121.412 92.964) (end 115.944 92.964) (width 0.25) (layer "F.Cu") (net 4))
 (segment (start 127.762 96.012) (end 124.46 96.012) (width 0.25) (layer "F.Cu") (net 4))
 (segment (start 135.892 89.684) (end 135.892 90.284) (width 0.25) (layer "F.Cu") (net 4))
 (segment (start 134.874 93.726) (end 130.048 93.726) (width 0.25) (layer "F.Cu") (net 4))
 (segment (start 136.74575 94.869) (end 140.105 91.50975) (width 0.25) (layer "F.Cu") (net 4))
 (segment (start 136.055 94.869) (end 135.44575 94.25975) (width 0.25) (layer "F.Cu") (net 4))
 (segment (start 135.892 89.684) (end 136.425 89.684) (width 0.25) (layer "F.Cu") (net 4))
 (segment (start 116.853 95.905) (end 114.928 93.98) (width 0.25) (layer "F.Cu") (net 4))
 (segment (start 116.853 97.135) (end 116.853 95.905) (width 0.25) (layer "F.Cu") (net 4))
 (segment (start 140.105 91.50975) (end 140.105 89.354) (width 0.25) (layer "F.Cu") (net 4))
 (segment (start 115.944 92.964) (end 114.928 93.98) (width 0.25) (layer "F.Cu") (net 4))
 (segment (start 136.055 94.869) (end 136.74575 94.869) (width 0.25) (layer "F.Cu") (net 4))
 (segment (start 135.40775 94.25975) (end 134.874 93.726) (width 0.25) (layer "F.Cu") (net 4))
 (segment (start 136.425 89.684) (end 138.43 87.679) (width 0.25) (layer "F.Cu") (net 4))
 (segment (start 115.824 99.06) (end 114.928 99.06) (width 0.25) (layer "F.Cu") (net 4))
 (segment (start 130.645 94.869) (end 129.667 94.869) (width 0.25) (layer "F.Cu") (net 10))
 (segment (start 128.016 96.52) (end 119.728 96.52) (width 0.25) (layer "F.Cu") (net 10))
 (segment (start 129.667 94.869) (end 128.016 96.52) (width 0.25) (layer "F.Cu") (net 10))
 (segment (start 131.568 89.084) (end 132.842 89.084) (width 0.25) (layer "F.Cu") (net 2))
 (segment (start 132.842 89.084) (end 132.842 89.684) (width 0.25) (layer "F.Cu") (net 2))
 (segment (start 128.966 89.154) (end 130.302 87.818) (width 0.25) (layer "F.Cu") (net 2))
 (segment (start 130.302 87.818) (end 131.568 89.084) (width 0.25) (layer "F.Cu") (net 2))
 (segment (start 127.692 89.154) (end 128.966 89.154) (width 0.25) (layer "F.Cu") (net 2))
 (segment (start 127.528 86.918) (end 125.292 89.154) (width 0.25) (layer "F.Cu") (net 16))
 (segment (start 132.284 86.918) (end 127.528 86.918) (width 0.25) (layer "F.Cu") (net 16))
 (segment (start 138.176 81.026) (end 132.284 86.918) (width 0.25) (layer "F.Cu") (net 16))
 (segment (start 129.921 97.409) (end 128.27 99.06) (width 0.25) (layer "F.Cu") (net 12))
 (segment (start 130.645 97.409) (end 129.921 97.409) (width 0.25) (layer "F.Cu") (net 12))
 (segment (start 128.27 99.06) (end 119.728 99.06) (width 0.25) (layer "F.Cu") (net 12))
 (segment (start 136.055 97.409) (end 134.493 97.409) (width 0.25) (layer "F.Cu") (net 9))
 (segment (start 112.553 88.615) (end 115.824 85.344) (width 0.25) (layer "F.Cu") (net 9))
 (segment (start 134.493 97.409) (end 131.667 100.235) (width 0.25) (layer "F.Cu") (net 9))
 (segment (start 112.816604 100.235) (end 112.553 99.971396) (width 0.25) (layer "F.Cu") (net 9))
 (segment (start 131.667 100.235) (end 112.816604 100.235) (width 0.25) (layer "F.Cu") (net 9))
 (segment (start 112.553 99.971396) (end 112.553 88.615) (width 0.25) (layer "F.Cu") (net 9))
 (segment (start 140.716 81.216) (end 139.351 79.851) (width 0.25) (layer "F.Cu") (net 8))
 (segment (start 139.351 79.851) (end 128.937 79.851) (width 0.25) (layer "F.Cu") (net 8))
 (segment (start 136.055 96.139) (end 136.74575 96.139) (width 0.25) (layer "F.Cu") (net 8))
 (segment (start 140.716 92.16875) (end 140.716 81.216) (width 0.25) (layer "F.Cu") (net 8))
 (segment (start 128.937 79.851) (end 123.444 85.344) (width 0.25) (layer "F.Cu") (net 8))
 (segment (start 136.74575 96.139) (end 140.716 92.16875) (width 0.25) (layer "F.Cu") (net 8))
 (segment (start 130.645 96.139) (end 130.92736 96.139) (width 0.25) (layer "F.Cu") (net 11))
 (segment (start 117.803 95.905) (end 117.803 97.245) (width 0.25) (layer "F.Cu") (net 11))
 (segment (start 119.728 93.98) (end 117.803 95.905) (width 0.25) (layer "F.Cu") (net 11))
 (segment (start 128.307 97.245) (end 129.094802 96.457198) (width 0.25) (layer "F.Cu") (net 11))
 (segment (start 117.803 97.245) (end 128.307 97.245) (width 0.25) (layer "F.Cu") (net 11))
 (segment (start 129.094802 96.457198) (end 130.326802 96.457198) (width 0.25) (layer "F.Cu") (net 11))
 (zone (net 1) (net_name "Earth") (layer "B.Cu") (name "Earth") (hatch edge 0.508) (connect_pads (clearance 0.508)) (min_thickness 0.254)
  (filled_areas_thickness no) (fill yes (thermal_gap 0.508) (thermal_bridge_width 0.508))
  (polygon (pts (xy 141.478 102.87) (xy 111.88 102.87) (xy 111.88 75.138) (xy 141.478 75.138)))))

